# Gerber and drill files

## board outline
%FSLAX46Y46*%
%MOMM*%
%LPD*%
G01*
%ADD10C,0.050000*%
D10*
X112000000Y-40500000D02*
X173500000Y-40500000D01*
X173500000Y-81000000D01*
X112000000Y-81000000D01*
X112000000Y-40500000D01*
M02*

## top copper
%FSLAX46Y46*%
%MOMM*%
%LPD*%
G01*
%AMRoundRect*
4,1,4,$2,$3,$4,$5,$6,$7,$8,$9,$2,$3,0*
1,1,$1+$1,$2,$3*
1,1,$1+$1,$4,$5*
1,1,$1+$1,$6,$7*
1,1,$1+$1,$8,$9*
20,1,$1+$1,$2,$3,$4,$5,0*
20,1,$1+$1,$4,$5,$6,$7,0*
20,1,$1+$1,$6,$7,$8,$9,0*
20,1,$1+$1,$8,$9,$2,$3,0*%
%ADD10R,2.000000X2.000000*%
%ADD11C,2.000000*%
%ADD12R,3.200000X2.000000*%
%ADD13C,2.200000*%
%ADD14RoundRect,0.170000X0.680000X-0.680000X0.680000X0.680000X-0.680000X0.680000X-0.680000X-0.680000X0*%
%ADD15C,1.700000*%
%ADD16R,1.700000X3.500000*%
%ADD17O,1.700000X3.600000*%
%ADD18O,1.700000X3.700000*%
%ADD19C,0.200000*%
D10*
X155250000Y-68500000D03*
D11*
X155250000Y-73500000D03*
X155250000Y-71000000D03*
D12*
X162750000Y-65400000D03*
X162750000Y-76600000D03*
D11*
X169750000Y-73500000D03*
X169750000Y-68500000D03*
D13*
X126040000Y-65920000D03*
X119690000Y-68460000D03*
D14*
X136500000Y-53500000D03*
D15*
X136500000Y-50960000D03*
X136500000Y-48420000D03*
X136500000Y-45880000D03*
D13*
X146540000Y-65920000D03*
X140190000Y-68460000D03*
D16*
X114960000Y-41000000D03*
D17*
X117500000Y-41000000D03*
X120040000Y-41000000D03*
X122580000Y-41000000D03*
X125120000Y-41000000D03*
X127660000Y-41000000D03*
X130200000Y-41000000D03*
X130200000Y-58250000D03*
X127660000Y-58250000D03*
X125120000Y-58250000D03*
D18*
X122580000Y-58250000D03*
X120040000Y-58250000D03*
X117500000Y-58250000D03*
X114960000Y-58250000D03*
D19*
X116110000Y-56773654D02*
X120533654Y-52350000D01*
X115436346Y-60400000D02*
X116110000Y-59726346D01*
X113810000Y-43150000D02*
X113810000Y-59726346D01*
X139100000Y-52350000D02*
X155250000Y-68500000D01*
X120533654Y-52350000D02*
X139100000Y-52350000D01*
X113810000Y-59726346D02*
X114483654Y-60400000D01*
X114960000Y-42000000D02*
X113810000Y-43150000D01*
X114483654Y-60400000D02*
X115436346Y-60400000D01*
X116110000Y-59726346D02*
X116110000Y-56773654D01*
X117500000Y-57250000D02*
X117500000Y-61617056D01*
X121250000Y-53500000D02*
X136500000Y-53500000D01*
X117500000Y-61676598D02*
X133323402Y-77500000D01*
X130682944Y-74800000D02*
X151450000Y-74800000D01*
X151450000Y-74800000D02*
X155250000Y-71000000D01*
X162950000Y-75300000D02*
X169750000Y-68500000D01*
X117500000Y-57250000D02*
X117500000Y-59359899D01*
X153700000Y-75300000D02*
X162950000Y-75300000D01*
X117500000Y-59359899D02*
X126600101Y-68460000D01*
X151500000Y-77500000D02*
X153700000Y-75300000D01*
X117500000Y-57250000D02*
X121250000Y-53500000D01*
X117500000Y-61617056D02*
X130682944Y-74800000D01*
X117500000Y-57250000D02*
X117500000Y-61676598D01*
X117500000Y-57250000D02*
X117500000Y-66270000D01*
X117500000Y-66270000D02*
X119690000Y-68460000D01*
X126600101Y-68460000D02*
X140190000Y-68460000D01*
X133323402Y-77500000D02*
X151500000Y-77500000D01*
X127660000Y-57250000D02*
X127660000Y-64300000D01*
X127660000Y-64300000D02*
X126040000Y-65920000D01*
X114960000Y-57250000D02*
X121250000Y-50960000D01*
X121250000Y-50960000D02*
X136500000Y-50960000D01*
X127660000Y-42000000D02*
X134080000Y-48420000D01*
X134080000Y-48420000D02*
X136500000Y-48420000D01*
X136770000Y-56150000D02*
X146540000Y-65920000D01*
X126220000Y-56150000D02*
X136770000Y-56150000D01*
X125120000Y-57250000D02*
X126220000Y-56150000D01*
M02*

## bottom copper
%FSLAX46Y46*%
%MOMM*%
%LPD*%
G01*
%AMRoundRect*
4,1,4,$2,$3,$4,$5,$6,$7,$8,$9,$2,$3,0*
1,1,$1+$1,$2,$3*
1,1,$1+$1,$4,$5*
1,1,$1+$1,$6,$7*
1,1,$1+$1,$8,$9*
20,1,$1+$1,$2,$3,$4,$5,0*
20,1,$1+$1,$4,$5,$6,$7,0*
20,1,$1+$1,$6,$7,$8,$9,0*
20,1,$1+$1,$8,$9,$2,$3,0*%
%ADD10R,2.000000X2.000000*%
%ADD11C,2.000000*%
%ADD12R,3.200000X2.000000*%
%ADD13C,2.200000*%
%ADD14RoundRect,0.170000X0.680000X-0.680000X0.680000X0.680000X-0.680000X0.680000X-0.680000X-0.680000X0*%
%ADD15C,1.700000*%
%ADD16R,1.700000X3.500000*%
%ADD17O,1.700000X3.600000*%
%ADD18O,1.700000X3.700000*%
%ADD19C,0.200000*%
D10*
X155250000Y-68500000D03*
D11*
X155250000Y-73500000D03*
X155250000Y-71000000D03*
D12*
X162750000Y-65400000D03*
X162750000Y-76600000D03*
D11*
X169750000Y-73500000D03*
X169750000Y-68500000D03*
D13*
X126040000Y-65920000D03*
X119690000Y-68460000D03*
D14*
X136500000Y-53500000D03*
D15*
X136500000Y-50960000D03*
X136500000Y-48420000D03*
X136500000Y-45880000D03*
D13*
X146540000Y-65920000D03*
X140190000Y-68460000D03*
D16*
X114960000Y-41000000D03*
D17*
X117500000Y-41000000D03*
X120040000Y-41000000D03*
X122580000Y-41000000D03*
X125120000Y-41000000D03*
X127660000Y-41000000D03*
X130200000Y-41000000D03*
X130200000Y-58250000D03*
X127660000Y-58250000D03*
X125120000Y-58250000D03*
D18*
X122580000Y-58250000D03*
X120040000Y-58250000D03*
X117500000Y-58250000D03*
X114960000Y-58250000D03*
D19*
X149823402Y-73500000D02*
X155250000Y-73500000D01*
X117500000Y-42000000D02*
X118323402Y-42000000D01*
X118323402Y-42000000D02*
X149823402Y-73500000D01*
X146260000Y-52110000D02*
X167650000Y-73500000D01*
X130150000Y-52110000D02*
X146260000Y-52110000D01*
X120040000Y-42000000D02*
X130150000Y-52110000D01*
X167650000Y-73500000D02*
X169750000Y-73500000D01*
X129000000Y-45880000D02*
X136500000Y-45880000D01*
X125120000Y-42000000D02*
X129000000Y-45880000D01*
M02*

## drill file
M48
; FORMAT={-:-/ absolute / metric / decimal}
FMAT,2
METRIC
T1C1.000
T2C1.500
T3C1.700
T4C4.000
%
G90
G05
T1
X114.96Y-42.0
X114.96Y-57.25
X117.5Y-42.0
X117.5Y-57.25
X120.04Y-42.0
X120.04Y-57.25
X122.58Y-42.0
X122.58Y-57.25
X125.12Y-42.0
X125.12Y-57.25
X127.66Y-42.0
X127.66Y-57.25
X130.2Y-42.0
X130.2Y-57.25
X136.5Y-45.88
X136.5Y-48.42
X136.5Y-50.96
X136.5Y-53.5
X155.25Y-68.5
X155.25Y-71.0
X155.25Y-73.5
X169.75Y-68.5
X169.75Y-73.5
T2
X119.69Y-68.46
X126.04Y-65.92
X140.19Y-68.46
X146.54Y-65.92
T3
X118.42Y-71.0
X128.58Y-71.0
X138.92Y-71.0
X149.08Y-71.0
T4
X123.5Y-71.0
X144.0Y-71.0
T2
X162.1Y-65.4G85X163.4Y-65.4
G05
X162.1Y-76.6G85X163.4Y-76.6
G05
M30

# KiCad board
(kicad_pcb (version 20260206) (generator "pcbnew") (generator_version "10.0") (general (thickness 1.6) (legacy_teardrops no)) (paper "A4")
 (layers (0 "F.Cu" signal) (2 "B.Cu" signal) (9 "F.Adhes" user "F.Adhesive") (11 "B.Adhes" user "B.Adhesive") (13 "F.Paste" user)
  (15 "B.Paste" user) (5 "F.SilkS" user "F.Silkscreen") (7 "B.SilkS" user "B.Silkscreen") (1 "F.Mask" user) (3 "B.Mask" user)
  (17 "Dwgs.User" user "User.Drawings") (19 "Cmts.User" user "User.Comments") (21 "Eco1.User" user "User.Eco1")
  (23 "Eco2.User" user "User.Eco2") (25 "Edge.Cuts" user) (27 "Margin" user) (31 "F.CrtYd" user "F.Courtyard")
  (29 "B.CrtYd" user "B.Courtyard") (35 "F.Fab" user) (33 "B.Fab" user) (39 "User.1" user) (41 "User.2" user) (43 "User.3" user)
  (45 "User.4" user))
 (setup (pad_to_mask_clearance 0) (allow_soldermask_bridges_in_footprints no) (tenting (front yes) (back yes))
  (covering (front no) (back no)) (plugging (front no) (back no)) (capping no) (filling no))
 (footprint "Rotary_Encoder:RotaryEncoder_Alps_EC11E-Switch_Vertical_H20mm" (layer "F.Cu") (at 155.25 68.5)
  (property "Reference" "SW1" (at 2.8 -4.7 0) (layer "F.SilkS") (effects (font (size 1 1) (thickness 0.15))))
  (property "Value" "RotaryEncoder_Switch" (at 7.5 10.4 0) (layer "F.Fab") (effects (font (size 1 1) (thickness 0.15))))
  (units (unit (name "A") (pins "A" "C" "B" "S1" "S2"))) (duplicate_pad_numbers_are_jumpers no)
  (pad "A" thru_hole rect (at 0 0) (size 2 2) (drill 1) (layers "*.Cu" "*.Mask") (remove_unused_layers no) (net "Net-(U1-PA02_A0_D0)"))
  (pad "B" thru_hole circle (at 0 5) (size 2 2) (drill 1) (layers "*.Cu" "*.Mask") (remove_unused_layers no) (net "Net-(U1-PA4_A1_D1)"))
  (pad "C" thru_hole circle (at 0 2.5) (size 2 2) (drill 1) (layers "*.Cu" "*.Mask") (remove_unused_layers no) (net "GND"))
  (pad "MP" thru_hole rect (at 7.5 -3.1) (size 3.2 2) (drill oval 2.8 1.5) (layers "*.Cu" "*.Mask") (remove_unused_layers no))
  (pad "MP" thru_hole rect (at 7.5 8.1) (size 3.2 2) (drill oval 2.8 1.5) (layers "*.Cu" "*.Mask") (remove_unused_layers no))
  (pad "S1" thru_hole circle (at 14.5 5) (size 2 2) (drill 1) (layers "*.Cu" "*.Mask") (remove_unused_layers no) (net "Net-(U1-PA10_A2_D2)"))
  (pad "S2" thru_hole circle (at 14.5 0) (size 2 2) (drill 1) (layers "*.Cu" "*.Mask") (remove_unused_layers no) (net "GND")))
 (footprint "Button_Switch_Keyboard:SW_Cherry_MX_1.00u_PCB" (layer "F.Cu") (at 126.04 65.92)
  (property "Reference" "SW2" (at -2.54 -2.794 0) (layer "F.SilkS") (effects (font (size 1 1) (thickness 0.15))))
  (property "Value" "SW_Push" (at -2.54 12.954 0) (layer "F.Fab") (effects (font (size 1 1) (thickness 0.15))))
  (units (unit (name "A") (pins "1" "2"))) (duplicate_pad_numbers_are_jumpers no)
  (pad "" np_thru_hole circle (at -7.62 5.08) (size 1.7 1.7) (drill 1.7) (layers "*.Cu" "*.Mask"))
  (pad "" np_thru_hole circle (at -2.54 5.08) (size 4 4) (drill 4) (layers "*.Cu" "*.Mask"))
  (pad "" np_thru_hole circle (at 2.54 5.08) (size 1.7 1.7) (drill 1.7) (layers "*.Cu" "*.Mask"))
  (pad "1" thru_hole circle (at 0 0) (size 2.2 2.2) (drill 1.5) (layers "*.Cu" "*.Mask") (remove_unused_layers no)
   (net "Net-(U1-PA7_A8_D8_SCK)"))
  (pad "2" thru_hole circle (at -6.35 2.54) (size 2.2 2.2) (drill 1.5) (layers "*.Cu" "*.Mask") (remove_unused_layers no) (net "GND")))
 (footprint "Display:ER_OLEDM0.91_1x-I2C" (layer "F.Cu") (at 136.5 53.5 90)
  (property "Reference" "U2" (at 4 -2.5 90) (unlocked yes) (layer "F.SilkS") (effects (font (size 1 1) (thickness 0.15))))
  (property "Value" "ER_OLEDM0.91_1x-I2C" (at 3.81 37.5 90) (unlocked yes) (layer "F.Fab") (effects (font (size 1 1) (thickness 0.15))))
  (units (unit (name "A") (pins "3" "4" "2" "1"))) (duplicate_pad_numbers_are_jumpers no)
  (pad "1" thru_hole roundrect (at 0 0 90) (size 1.7 1.7) (drill 1) (layers "*.Cu" "*.Mask") (remove_unused_layers no)
   (roundrect_rratio 0.1) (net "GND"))
  (pad "2" thru_hole circle (at 2.54 0 90) (size 1.7 1.7) (drill 1) (layers "*.Cu" "*.Mask") (remove_unused_layers no) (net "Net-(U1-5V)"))
  (pad "3" thru_hole circle (at 5.08 0 90) (size 1.7 1.7) (drill 1) (layers "*.Cu" "*.Mask") (remove_unused_layers no)
   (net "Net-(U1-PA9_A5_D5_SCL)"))
  (pad "4" thru_hole circle (at 7.62 0 90) (size 1.7 1.7) (drill 1) (layers "*.Cu" "*.Mask") (remove_unused_layers no)
   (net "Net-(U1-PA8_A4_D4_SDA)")))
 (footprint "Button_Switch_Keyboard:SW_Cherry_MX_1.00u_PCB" (layer "F.Cu") (at 146.54 65.92)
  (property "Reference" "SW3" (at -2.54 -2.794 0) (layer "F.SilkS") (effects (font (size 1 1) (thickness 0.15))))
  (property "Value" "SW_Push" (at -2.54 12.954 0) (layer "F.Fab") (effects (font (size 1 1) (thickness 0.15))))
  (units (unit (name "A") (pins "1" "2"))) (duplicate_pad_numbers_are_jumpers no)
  (pad "" np_thru_hole circle (at -7.62 5.08) (size 1.7 1.7) (drill 1.7) (layers "*.Cu" "*.Mask"))
  (pad "" np_thru_hole circle (at -2.54 5.08) (size 4 4) (drill 4) (layers "*.Cu" "*.Mask"))
  (pad "" np_thru_hole circle (at 2.54 5.08) (size 1.7 1.7) (drill 1.7) (layers "*.Cu" "*.Mask"))
  (pad "1" thru_hole circle (at 0 0) (size 2.2 2.2) (drill 1.5) (layers "*.Cu" "*.Mask") (remove_unused_layers no)
   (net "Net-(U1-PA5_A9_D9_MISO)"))
  (pad "2" thru_hole circle (at -6.35 2.54) (size 2.2 2.2) (drill 1.5) (layers "*.Cu" "*.Mask") (remove_unused_layers no) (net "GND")))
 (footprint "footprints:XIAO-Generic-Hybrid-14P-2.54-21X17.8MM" (layer "B.Cu") (at 122.58 49.625 -90)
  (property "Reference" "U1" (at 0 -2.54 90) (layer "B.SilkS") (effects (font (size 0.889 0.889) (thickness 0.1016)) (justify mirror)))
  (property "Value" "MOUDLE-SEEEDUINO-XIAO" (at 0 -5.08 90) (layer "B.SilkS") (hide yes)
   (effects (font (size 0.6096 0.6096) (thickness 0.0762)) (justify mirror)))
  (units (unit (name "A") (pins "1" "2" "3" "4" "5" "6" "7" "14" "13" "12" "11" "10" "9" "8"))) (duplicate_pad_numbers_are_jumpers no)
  (pad "1" thru_hole rect (at -7.625 7.62 270) (size 3.5 1.7) (drill 1 (offset -1 0)) (layers "*.Cu" "*.Mask") (remove_unused_layers no)
   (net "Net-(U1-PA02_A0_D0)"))
  (pad "2" thru_hole oval (at -7.625 5.08 270) (size 3.6 1.7) (drill 1 (offset -1 0)) (layers "*.Cu" "*.Mask") (remove_unused_layers no)
   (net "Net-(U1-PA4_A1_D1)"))
  (pad "3" thru_hole oval (at -7.625 2.54 270) (size 3.6 1.7) (drill 1 (offset -1 0)) (layers "*.Cu" "*.Mask") (remove_unused_layers no)
   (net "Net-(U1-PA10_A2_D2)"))
  (pad "4" thru_hole oval (at -7.625 0 270) (size 3.6 1.7) (drill 1 (offset -1 0)) (layers "*.Cu" "*.Mask") (remove_unused_layers no)
   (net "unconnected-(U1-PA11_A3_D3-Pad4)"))
  (pad "5" thru_hole oval (at -7.625 -2.54 270) (size 3.6 1.7) (drill 1 (offset -1 0)) (layers "*.Cu" "*.Mask") (remove_unused_layers no)
   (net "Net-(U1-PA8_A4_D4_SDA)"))
  (pad "6" thru_hole oval (at -7.625 -5.08 90) (size 3.6 1.7) (drill 1 (offset 1 0)) (layers "*.Cu" "*.Mask") (remove_unused_layers no)
   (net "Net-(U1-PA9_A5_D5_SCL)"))
  (pad "7" thru_hole oval (at -7.625 -7.62 270) (size 3.6 1.7) (drill 1 (offset -1 0)) (layers "*.Cu" "*.Mask") (remove_unused_layers no)
   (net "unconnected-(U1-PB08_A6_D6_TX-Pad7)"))
  (pad "8" thru_hole oval (at 7.625 -7.62 270) (size 3.6 1.7) (drill 1 (offset 1 0)) (layers "*.Cu" "*.Mask") (remove_unused_layers no)
   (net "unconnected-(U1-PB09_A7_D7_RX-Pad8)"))
  (pad "9" thru_hole oval (at 7.625 -5.08 270) (size 3.6 1.7) (drill 1 (offset 1 0)) (layers "*.Cu" "*.Mask") (remove_unused_layers no)
   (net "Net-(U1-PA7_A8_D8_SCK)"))
  (pad "10" thru_hole oval (at 7.625 -2.54 270) (size 3.6 1.7) (drill 1 (offset 1 0)) (layers "*.Cu" "*.Mask") (remove_unused_layers no)
   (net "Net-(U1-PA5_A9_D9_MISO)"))
  (pad "11" thru_hole oval (at 7.625 0 270) (size 3.7 1.7) (drill 1 (offset 1 0)) (layers "*.Cu" "*.Mask") (remove_unused_layers no)
   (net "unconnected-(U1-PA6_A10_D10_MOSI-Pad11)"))
  (pad "12" thru_hole oval (at 7.625 2.54 270) (size 3.7 1.7) (drill 1 (offset 1 0)) (layers "*.Cu" "*.Mask") (remove_unused_layers no)
   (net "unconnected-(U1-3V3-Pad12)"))
  (pad "13" thru_hole oval (at 7.625 5.08 270) (size 3.7 1.7) (drill 1 (offset 1 0)) (layers "*.Cu" "*.Mask") (remove_unused_layers no)
   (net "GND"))
  (pad "14" thru_hole oval (at 7.625 7.62 270) (size 3.7 1.7) (drill 1 (offset 1 0)) (layers "*.Cu" "*.Mask") (remove_unused_layers no)
   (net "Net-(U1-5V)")))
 (gr_rect (start 112 40.5) (end 173.5 81) (stroke (width 0.05) (type default)) (fill no) (layer "Edge.Cuts"))
 (segment (start 116.11 56.773654) (end 120.533654 52.35) (width 0.2) (layer "F.Cu") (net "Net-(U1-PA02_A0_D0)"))
 (segment (start 115.436346 60.4) (end 116.11 59.726346) (width 0.2) (layer "F.Cu") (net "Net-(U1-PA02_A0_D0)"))
 (segment (start 113.81 43.15) (end 113.81 59.726346) (width 0.2) (layer "F.Cu") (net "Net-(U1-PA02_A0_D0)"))
 (segment (start 139.1 52.35) (end 155.25 68.5) (width 0.2) (layer "F.Cu") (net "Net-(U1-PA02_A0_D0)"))
 (segment (start 120.533654 52.35) (end 139.1 52.35) (width 0.2) (layer "F.Cu") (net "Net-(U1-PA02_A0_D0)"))
 (segment (start 113.81 59.726346) (end 114.483654 60.4) (width 0.2) (layer "F.Cu") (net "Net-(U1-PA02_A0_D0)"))
 (segment (start 114.96 42) (end 113.81 43.15) (width 0.2) (layer "F.Cu") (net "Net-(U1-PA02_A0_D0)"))
 (segment (start 114.483654 60.4) (end 115.436346 60.4) (width 0.2) (layer "F.Cu") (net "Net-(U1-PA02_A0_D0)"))
 (segment (start 116.11 59.726346) (end 116.11 56.773654) (width 0.2) (layer "F.Cu") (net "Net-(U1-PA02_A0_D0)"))
 (segment (start 149.823402 73.5) (end 155.25 73.5) (width 0.2) (layer "B.Cu") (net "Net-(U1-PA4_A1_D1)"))
 (segment (start 117.5 42) (end 118.323402 42) (width 0.2) (layer "B.Cu") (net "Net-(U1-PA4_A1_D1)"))
 (segment (start 118.323402 42) (end 149.823402 73.5) (width 0.2) (layer "B.Cu") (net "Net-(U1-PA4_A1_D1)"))
 (segment (start 117.5 57.25) (end 117.5 61.617056) (width 0.2) (layer "F.Cu") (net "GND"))
 (segment (start 121.25 53.5) (end 136.5 53.5) (width 0.2) (layer "F.Cu") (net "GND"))
 (segment (start 117.5 61.676598) (end 133.323402 77.5) (width 0.2) (layer "F.Cu") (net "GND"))
 (segment (start 130.682944 74.8) (end 151.45 74.8) (width 0.2) (layer "F.Cu") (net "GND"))
 (segment (start 151.45 74.8) (end 155.25 71) (width 0.2) (layer "F.Cu") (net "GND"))
 (segment (start 162.95 75.3) (end 169.75 68.5) (width 0.2) (layer "F.Cu") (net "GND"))
 (segment (start 117.5 57.25) (end 117.5 59.359899) (width 0.2) (layer "F.Cu") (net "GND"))
 (segment (start 153.7 75.3) (end 162.95 75.3) (width 0.2) (layer "F.Cu") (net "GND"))
 (segment (start 117.5 59.359899) (end 126.600101 68.46) (width 0.2) (layer "F.Cu") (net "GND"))
 (segment (start 151.5 77.5) (end 153.7 75.3) (width 0.2) (layer "F.Cu") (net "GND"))
 (segment (start 117.5 57.25) (end 121.25 53.5) (width 0.2) (layer "F.Cu") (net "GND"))
 (segment (start 117.5 61.617056) (end 130.682944 74.8) (width 0.2) (layer "F.Cu") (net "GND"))
 (segment (start 117.5 57.25) (end 117.5 61.676598) (width 0.2) (layer "F.Cu") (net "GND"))
 (segment (start 117.5 57.25) (end 117.5 66.27) (width 0.2) (layer "F.Cu") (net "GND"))
 (segment (start 117.5 66.27) (end 119.69 68.46) (width 0.2) (layer "F.Cu") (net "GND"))
 (segment (start 126.600101 68.46) (end 140.19 68.46) (width 0.2) (layer "F.Cu") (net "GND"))
 (segment (start 133.323402 77.5) (end 151.5 77.5) (width 0.2) (layer "F.Cu") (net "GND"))
 (segment (start 146.26 52.11) (end 167.65 73.5) (width 0.2) (layer "B.Cu") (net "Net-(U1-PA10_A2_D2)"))
 (segment (start 130.15 52.11) (end 146.26 52.11) (width 0.2) (layer "B.Cu") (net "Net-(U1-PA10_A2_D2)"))
 (segment (start 120.04 42) (end 130.15 52.11) (width 0.2) (layer "B.Cu") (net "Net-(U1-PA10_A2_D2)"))
 (segment (start 167.65 73.5) (end 169.75 73.5) (width 0.2) (layer "B.Cu") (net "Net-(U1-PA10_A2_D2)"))
 (segment (start 127.66 57.25) (end 127.66 64.3) (width 0.2) (layer "F.Cu") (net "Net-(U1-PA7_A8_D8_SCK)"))
 (segment (start 127.66 64.3) (end 126.04 65.92) (width 0.2) (layer "F.Cu") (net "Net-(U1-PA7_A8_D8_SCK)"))
 (segment (start 114.96 57.25) (end 121.25 50.96) (width 0.2) (layer "F.Cu") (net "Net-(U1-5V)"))
 (segment (start 121.25 50.96) (end 136.5 50.96) (width 0.2) (layer "F.Cu") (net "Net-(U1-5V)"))
 (segment (start 127.66 42) (end 134.08 48.42) (width 0.2) (layer "F.Cu") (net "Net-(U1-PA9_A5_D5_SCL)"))
 (segment (start 134.08 48.42) (end 136.5 48.42) (width 0.2) (layer "F.Cu") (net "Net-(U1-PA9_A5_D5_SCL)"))
 (segment (start 129 45.88) (end 136.5 45.88) (width 0.2) (layer "B.Cu") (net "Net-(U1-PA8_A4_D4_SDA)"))
 (segment (start 125.12 42) (end 129 45.88) (width 0.2) (layer "B.Cu") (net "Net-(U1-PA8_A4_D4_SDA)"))
 (segment (start 136.77 56.15) (end 146.54 65.92) (width 0.2) (layer "F.Cu") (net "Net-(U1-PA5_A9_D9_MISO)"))
 (segment (start 126.22 56.15) (end 136.77 56.15) (width 0.2) (layer "F.Cu") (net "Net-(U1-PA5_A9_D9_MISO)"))
 (segment (start 125.12 57.25) (end 126.22 56.15) (width 0.2) (layer "F.Cu") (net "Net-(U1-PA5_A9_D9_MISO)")))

